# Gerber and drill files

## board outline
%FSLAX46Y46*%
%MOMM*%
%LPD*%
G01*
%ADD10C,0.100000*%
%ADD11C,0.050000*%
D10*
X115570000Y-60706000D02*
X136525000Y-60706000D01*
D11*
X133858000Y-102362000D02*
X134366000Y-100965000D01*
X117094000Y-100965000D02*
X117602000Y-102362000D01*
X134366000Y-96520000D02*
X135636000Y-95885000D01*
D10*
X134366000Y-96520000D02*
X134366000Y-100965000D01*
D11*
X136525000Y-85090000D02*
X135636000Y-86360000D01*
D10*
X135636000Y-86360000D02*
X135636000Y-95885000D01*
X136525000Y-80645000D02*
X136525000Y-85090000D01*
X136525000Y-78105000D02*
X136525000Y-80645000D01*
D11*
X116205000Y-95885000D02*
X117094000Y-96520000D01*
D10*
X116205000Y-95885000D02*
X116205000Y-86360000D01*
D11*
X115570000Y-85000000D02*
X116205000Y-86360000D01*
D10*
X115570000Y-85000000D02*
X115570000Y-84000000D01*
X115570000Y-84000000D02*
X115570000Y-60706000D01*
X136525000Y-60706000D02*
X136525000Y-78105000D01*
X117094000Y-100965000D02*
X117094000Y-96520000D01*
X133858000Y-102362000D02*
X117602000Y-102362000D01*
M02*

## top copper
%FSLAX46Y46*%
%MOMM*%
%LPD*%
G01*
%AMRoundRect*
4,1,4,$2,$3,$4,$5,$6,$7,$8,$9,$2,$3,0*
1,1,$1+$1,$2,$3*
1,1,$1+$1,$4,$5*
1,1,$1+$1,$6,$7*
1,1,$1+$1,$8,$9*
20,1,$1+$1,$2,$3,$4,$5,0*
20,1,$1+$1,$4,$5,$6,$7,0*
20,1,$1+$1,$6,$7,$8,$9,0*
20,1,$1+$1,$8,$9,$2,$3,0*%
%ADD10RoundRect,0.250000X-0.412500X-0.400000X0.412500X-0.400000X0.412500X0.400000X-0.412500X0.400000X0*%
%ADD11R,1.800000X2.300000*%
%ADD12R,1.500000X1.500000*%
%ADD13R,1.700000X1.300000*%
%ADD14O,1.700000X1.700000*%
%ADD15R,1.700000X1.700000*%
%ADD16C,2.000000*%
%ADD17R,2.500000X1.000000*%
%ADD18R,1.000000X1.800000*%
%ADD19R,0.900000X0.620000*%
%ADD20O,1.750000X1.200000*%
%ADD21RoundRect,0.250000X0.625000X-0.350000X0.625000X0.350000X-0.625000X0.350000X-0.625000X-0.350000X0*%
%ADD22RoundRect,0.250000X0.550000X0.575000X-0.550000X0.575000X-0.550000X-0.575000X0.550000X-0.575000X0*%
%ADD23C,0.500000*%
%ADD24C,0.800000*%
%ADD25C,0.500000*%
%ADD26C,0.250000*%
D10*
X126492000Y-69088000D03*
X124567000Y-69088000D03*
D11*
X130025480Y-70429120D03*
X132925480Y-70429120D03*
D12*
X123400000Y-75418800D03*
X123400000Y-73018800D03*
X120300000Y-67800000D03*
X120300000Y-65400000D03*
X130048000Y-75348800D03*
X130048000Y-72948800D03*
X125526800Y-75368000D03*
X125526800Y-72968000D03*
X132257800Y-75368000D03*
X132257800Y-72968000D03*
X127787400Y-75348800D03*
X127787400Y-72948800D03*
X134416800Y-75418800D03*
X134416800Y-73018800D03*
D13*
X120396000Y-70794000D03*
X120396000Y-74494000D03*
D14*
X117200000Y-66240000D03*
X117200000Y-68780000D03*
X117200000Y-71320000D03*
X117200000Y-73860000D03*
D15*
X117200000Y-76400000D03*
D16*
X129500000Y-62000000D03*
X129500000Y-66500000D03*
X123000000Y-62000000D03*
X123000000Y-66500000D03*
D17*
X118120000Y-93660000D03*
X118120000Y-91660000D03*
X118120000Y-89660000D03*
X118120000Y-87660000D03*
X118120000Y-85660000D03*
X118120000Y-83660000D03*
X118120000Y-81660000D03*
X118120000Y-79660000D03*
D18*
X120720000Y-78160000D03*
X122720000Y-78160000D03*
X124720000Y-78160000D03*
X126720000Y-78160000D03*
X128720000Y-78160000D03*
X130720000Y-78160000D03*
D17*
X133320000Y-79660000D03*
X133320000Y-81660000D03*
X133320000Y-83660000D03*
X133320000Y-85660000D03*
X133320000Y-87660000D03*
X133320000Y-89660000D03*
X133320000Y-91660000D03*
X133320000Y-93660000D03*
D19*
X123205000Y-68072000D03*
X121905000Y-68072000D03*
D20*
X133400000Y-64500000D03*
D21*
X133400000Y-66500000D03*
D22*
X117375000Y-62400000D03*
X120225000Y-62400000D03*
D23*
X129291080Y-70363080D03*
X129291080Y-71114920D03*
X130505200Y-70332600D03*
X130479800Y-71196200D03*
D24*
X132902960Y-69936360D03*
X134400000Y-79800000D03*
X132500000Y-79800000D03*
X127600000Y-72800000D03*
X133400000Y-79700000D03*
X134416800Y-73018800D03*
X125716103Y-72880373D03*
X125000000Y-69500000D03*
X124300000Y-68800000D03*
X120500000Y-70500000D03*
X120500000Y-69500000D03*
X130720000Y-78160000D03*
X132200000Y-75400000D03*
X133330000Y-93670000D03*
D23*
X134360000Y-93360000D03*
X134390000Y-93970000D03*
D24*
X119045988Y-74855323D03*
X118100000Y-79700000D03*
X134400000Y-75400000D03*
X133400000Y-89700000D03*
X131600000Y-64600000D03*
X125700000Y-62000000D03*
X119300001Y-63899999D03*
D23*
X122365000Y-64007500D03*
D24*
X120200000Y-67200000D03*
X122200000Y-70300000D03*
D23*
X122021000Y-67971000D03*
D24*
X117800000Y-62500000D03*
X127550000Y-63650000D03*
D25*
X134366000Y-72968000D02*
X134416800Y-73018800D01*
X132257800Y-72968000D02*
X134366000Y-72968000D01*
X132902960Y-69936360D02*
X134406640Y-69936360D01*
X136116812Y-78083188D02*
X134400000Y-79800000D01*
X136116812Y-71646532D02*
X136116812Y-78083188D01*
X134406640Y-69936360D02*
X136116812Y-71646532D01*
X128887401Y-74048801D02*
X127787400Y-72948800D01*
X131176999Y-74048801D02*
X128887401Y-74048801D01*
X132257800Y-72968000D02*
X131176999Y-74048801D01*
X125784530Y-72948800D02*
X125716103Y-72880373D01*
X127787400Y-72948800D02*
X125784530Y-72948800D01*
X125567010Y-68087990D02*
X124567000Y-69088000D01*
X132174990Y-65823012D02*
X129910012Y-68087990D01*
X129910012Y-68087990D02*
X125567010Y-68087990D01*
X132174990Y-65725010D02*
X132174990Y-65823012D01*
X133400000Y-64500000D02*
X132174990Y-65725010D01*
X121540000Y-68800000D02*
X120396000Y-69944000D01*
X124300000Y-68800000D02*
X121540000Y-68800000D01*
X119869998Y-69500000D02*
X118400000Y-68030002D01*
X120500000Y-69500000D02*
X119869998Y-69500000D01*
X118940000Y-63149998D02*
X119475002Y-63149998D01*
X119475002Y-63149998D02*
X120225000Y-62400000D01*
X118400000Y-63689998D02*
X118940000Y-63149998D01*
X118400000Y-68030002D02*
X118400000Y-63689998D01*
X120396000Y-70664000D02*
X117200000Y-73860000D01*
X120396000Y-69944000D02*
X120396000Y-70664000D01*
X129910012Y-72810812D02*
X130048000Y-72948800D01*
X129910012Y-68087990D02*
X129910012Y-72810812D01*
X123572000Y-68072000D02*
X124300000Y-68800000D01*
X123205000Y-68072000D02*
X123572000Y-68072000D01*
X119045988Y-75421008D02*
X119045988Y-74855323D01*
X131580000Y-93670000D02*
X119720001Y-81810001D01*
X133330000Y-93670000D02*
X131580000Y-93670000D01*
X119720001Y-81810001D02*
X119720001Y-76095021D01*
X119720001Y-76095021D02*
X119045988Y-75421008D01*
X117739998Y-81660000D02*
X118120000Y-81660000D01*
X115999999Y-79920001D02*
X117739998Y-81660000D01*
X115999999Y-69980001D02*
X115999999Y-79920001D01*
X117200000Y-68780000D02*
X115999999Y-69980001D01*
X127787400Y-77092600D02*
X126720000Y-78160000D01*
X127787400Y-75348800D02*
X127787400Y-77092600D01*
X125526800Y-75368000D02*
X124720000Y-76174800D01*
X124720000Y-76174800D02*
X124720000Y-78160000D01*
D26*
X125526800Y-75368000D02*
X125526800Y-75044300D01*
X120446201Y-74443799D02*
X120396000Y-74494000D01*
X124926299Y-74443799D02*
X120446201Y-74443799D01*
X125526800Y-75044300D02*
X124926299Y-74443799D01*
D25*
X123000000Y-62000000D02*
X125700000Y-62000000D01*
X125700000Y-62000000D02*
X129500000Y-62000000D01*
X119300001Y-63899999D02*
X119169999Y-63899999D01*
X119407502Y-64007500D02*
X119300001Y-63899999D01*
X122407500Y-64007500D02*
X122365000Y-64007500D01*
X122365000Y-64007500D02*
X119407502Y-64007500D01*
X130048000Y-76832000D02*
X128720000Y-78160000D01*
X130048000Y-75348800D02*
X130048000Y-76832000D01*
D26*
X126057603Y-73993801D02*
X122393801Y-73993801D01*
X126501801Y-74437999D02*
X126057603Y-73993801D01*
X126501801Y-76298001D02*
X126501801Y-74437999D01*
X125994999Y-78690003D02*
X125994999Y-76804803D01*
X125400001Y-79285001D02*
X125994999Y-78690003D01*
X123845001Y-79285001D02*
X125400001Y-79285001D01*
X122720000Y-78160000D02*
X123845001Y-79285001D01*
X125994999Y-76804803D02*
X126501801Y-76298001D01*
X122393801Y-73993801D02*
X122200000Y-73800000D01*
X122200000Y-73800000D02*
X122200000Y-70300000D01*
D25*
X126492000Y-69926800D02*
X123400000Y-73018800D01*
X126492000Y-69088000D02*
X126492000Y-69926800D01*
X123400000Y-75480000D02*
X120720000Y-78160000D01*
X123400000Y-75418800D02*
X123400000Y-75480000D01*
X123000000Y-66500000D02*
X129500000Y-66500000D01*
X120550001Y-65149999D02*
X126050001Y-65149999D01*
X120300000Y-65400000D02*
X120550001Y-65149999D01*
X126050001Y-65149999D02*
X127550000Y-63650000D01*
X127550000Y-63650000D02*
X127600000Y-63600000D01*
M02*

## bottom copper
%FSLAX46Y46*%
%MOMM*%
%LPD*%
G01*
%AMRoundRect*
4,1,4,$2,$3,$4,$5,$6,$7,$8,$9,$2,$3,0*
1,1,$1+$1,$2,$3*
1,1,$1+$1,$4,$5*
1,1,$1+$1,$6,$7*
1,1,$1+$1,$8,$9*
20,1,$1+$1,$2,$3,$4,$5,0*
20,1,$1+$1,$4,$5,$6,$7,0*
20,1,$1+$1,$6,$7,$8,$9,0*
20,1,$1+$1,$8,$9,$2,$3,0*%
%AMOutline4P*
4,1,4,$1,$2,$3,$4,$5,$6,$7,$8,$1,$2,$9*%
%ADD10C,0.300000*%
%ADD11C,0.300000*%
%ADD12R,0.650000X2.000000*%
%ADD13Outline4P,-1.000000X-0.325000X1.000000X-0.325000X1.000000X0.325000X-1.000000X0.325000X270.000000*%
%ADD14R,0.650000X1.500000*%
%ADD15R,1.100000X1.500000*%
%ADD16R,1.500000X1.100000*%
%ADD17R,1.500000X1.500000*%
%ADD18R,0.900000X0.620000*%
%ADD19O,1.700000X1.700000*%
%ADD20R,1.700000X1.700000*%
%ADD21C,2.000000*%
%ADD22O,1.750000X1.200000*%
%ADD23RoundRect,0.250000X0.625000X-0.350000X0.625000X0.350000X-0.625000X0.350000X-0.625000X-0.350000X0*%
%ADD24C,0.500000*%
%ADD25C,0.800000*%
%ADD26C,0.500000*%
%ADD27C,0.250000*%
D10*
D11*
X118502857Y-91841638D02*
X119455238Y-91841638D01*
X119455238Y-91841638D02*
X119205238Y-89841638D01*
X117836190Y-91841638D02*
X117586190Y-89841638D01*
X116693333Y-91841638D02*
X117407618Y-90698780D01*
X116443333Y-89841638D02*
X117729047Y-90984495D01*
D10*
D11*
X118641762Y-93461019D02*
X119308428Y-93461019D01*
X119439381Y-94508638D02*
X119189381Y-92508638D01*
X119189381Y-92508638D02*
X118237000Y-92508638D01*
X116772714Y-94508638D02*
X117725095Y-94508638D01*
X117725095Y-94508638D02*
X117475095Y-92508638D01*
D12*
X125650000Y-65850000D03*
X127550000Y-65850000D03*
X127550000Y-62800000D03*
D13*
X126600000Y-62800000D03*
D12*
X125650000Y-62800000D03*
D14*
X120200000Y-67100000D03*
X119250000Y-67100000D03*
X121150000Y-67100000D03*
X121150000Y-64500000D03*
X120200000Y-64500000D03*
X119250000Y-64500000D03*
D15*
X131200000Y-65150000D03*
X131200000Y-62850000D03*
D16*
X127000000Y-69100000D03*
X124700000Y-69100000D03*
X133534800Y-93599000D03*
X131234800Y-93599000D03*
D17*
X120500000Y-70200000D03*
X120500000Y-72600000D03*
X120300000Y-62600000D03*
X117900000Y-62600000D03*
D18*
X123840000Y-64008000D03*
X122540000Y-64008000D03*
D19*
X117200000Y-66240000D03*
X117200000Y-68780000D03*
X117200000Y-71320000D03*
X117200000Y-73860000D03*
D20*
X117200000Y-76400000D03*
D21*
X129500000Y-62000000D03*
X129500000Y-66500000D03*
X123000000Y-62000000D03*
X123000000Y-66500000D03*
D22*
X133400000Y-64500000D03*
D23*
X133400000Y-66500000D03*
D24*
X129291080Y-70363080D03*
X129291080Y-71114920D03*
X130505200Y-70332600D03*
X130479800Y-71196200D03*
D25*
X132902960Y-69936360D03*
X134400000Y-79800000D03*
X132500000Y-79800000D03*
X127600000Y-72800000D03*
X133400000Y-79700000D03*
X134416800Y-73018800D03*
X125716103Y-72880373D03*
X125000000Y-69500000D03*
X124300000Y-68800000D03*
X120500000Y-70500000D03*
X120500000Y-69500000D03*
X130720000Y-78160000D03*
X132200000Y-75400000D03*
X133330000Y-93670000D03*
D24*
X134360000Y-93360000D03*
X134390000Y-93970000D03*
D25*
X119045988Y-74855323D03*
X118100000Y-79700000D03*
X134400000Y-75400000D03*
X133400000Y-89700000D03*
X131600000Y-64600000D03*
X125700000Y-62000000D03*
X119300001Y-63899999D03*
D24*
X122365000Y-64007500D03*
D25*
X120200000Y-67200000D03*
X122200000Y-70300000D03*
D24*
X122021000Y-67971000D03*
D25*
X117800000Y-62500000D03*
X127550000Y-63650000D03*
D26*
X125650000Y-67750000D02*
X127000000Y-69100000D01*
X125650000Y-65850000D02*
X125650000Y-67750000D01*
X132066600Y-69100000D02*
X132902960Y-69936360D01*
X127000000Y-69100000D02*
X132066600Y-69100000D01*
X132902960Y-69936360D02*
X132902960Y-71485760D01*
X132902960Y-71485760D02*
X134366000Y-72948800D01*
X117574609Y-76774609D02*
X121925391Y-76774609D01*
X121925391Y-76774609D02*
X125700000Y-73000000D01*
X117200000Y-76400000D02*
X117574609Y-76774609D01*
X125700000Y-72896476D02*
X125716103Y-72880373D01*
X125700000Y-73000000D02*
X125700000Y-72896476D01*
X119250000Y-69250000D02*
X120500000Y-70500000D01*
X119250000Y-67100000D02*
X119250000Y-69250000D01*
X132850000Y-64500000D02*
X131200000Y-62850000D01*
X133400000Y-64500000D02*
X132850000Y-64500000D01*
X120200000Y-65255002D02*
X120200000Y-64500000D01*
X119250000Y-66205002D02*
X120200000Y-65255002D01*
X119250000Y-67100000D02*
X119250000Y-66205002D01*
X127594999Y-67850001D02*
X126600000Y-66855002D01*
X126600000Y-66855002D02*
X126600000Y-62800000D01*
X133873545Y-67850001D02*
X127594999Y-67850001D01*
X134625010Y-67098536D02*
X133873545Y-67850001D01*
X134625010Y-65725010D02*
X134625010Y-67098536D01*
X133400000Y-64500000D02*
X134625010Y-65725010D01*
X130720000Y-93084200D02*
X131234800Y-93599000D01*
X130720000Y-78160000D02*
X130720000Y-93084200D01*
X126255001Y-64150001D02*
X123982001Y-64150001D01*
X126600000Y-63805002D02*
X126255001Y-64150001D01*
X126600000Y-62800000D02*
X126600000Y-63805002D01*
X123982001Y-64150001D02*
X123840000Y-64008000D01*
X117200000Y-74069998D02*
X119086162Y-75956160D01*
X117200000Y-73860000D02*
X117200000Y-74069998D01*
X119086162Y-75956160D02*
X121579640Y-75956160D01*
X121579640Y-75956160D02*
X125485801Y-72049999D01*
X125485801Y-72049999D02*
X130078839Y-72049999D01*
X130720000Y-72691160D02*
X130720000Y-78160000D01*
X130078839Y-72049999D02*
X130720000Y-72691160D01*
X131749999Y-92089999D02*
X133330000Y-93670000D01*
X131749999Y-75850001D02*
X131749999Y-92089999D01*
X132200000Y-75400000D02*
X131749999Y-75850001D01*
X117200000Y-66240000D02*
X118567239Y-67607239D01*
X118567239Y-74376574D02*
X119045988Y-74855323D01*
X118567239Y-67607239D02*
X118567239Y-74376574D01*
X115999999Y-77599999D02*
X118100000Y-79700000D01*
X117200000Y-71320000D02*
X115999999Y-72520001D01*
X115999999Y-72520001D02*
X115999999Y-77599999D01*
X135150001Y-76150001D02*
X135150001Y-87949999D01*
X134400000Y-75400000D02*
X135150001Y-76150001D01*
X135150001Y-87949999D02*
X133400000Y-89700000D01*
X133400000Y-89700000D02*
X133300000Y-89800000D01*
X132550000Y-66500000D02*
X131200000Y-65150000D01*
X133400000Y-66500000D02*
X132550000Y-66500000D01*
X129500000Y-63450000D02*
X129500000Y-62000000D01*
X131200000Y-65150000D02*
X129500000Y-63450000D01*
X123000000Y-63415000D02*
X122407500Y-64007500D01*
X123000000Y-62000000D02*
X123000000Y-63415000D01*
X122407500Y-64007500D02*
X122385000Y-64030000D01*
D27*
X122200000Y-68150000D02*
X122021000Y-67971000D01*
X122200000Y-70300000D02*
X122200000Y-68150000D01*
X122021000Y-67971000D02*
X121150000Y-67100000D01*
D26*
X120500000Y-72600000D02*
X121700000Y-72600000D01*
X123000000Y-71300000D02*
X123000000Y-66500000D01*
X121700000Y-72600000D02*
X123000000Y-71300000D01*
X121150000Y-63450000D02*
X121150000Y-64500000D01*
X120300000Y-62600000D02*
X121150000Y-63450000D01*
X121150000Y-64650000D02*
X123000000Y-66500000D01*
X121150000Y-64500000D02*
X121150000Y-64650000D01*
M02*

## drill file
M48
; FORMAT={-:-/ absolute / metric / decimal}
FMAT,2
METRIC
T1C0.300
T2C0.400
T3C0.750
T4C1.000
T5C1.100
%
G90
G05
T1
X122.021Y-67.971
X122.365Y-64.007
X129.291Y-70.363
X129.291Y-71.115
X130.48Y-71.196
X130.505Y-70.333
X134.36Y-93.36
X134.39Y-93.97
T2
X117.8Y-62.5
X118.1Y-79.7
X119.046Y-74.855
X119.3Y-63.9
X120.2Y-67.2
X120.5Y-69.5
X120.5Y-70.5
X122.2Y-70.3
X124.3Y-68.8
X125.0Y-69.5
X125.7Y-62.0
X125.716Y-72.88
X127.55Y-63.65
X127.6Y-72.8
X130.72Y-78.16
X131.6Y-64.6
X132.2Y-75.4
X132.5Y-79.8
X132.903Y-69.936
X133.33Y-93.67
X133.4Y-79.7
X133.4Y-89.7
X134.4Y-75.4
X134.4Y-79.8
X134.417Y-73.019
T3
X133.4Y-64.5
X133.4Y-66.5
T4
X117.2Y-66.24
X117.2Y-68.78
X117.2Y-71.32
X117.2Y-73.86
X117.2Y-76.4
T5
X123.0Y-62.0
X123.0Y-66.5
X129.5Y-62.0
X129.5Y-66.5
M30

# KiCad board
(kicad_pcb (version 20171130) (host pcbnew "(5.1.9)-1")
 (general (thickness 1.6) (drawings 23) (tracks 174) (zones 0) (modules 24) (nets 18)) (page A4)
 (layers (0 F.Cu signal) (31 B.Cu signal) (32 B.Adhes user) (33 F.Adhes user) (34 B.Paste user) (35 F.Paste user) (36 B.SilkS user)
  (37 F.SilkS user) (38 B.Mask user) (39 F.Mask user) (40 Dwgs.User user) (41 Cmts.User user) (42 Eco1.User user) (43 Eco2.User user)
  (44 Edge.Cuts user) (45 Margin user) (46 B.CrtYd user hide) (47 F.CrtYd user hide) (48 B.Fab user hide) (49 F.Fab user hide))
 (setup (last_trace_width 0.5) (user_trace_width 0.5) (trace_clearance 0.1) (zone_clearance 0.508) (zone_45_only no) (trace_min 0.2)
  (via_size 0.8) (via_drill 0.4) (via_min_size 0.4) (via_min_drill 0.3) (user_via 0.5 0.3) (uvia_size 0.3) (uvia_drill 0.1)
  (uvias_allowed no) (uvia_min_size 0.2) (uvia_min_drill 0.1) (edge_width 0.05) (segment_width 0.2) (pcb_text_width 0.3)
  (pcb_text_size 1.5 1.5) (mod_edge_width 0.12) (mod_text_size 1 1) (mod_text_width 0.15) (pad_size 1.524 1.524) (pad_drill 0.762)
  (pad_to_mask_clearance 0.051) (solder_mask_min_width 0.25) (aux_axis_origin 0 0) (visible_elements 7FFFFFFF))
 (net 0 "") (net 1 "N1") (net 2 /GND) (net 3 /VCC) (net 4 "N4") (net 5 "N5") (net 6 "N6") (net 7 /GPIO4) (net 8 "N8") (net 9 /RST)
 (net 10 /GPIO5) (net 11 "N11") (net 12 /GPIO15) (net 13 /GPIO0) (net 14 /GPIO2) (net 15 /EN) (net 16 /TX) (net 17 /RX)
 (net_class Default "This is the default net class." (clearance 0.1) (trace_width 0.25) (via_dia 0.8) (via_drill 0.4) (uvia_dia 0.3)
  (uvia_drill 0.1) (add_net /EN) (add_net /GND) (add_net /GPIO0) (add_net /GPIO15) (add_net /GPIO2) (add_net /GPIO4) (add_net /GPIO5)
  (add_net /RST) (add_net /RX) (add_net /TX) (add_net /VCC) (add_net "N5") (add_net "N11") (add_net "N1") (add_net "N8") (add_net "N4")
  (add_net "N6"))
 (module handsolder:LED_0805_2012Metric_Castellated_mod (layer F.Cu) (at 125.5295 69.088)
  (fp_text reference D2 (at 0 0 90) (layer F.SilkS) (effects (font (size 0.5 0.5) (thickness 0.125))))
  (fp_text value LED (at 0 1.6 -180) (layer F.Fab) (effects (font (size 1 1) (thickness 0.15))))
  (pad 2 smd roundrect (at 0.9625 0) (size 1.325 1.3) (layers F.Cu F.Paste F.Mask) (roundrect_rratio 0.1923076923076923) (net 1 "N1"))
  (pad 1 smd roundrect (at -0.9625 0) (size 1.325 1.3) (layers F.Cu F.Paste F.Mask) (roundrect_rratio 0.1923076923076923) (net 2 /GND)))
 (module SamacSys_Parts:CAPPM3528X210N (layer F.Cu) (at 131.47548 70.42912 180)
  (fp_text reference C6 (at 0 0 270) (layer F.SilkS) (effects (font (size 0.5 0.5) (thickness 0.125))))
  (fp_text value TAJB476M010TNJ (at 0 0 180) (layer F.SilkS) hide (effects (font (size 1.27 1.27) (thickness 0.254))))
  (pad 2 smd rect (at 1.45 0 180) (size 1.8 2.3) (layers F.Cu F.Paste F.Mask) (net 2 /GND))
  (pad 1 smd rect (at -1.45 0 180) (size 1.8 2.3) (layers F.Cu F.Paste F.Mask) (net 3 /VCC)))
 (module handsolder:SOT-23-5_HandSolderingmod (layer B.Cu) (at 126.6 64.35 270)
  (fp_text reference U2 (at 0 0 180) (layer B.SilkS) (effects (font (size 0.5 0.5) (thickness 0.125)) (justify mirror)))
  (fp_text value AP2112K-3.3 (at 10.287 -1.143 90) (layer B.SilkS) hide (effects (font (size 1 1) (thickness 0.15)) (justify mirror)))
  (pad 5 smd rect (at 1.5 0.95 270) (size 2 0.65) (layers B.Cu B.Paste B.Mask) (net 3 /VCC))
  (pad 4 smd rect (at 1.5 -0.95 270) (size 2 0.65) (layers B.Cu B.Paste B.Mask))
  (pad 3 smd rect (at -1.55 -0.95 270) (size 2 0.65) (layers B.Cu B.Paste B.Mask) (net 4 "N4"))
  (pad 2 smd trapezoid (at -1.55 0 270) (size 2 0.65) (layers B.Cu B.Paste B.Mask) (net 2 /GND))
  (pad 1 smd rect (at -1.55 0.95 270) (size 2 0.65) (layers B.Cu B.Paste B.Mask) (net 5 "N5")))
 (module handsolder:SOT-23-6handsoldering (layer B.Cu) (at 120.2 65.8 270)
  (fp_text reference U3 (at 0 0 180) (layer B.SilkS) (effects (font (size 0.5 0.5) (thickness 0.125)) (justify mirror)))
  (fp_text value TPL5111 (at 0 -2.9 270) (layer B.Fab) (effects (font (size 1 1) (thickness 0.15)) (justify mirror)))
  (pad 5 smd rect (at 1.3 0 270) (size 1.5 0.65) (layers B.Cu B.Paste B.Mask) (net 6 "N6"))
  (pad 6 smd rect (at 1.3 0.95 270) (size 1.5 0.65) (layers B.Cu B.Paste B.Mask) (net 2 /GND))
  (pad 4 smd rect (at 1.3 -0.95 270) (size 1.5 0.65) (layers B.Cu B.Paste B.Mask) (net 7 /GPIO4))
  (pad 3 smd rect (at -1.3 -0.95 270) (size 1.5 0.65) (layers B.Cu B.Paste B.Mask) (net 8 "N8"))
  (pad 2 smd rect (at -1.3 0 270) (size 1.5 0.65) (layers B.Cu B.Paste B.Mask) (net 2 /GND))
  (pad 1 smd rect (at -1.3 0.95 270) (size 1.5 0.65) (layers B.Cu B.Paste B.Mask) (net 5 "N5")))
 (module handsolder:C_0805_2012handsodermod (layer B.Cu) (at 131.2 64 270)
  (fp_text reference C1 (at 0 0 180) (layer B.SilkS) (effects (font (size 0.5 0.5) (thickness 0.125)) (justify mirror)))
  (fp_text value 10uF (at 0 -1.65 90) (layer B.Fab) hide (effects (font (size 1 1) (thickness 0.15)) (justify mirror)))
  (pad 2 smd rect (at 1.15 0 270) (size 1.5 1.1) (layers B.Cu B.Paste B.Mask) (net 5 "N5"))
  (pad 1 smd rect (at -1.15 0 270) (size 1.5 1.1) (layers B.Cu B.Paste B.Mask) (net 2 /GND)))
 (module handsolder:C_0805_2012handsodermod (layer B.Cu) (at 125.85 69.1)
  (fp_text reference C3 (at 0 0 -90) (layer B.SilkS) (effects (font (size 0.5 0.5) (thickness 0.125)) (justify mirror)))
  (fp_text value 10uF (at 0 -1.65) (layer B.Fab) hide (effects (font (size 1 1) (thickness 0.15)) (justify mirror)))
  (pad 2 smd rect (at 1.15 0) (size 1.5 1.1) (layers B.Cu B.Paste B.Mask) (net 3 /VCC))
  (pad 1 smd rect (at -1.15 0) (size 1.5 1.1) (layers B.Cu B.Paste B.Mask) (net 2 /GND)))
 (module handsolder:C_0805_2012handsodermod (layer B.Cu) (at 132.3848 93.599)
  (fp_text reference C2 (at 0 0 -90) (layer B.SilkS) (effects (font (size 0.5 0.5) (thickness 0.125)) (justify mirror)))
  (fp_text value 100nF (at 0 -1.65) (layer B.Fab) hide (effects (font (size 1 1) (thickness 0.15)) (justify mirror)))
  (pad 2 smd rect (at 1.15 0) (size 1.5 1.1) (layers B.Cu B.Paste B.Mask) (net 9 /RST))
  (pad 1 smd rect (at -1.15 0) (size 1.5 1.1) (layers B.Cu B.Paste B.Mask) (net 2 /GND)))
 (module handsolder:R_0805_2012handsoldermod (layer B.Cu) (at 120.5 71.4 90)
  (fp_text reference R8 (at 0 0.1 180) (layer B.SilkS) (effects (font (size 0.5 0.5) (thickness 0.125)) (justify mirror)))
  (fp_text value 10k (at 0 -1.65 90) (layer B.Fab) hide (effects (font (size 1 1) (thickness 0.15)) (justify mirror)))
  (pad 2 smd rect (at 1.2 0 90) (size 1.5 1.5) (layers B.Cu B.Paste B.Mask) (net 2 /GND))
  (pad 1 smd rect (at -1.2 0 90) (size 1.5 1.5) (layers B.Cu B.Paste B.Mask) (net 8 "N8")))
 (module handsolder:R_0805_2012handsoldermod (layer F.Cu) (at 123.4 74.2188 270)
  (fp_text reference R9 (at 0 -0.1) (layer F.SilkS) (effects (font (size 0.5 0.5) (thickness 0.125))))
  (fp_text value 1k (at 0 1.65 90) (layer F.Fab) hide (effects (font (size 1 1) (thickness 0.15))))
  (pad 2 smd rect (at 1.2 0 270) (size 1.5 1.5) (layers F.Cu F.Paste F.Mask) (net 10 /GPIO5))
  (pad 1 smd rect (at -1.2 0 270) (size 1.5 1.5) (layers F.Cu F.Paste F.Mask) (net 1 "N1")))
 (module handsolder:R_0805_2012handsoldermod (layer F.Cu) (at 120.3 66.6 270)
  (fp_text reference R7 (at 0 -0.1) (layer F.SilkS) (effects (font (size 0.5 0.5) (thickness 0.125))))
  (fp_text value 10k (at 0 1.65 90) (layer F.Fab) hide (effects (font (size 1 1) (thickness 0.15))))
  (pad 2 smd rect (at 1.2 0 270) (size 1.5 1.5) (layers F.Cu F.Paste F.Mask) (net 6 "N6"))
  (pad 1 smd rect (at -1.2 0 270) (size 1.5 1.5) (layers F.Cu F.Paste F.Mask) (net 4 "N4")))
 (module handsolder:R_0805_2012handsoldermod (layer B.Cu) (at 119.1 62.6)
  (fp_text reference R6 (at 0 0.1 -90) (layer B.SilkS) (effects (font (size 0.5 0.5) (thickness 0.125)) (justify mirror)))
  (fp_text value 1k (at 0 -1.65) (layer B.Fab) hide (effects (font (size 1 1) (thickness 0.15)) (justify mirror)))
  (pad 2 smd rect (at 1.2 0) (size 1.5 1.5) (layers B.Cu B.Paste B.Mask) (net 8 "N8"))
  (pad 1 smd rect (at -1.2 0) (size 1.5 1.5) (layers B.Cu B.Paste B.Mask) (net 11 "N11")))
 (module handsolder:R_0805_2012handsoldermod (layer F.Cu) (at 130.048 74.1488 270)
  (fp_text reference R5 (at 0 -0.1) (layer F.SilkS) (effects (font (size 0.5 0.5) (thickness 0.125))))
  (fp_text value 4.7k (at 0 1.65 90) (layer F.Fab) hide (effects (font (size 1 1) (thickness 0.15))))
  (pad 2 smd rect (at 1.2 0 270) (size 1.5 1.5) (layers F.Cu F.Paste F.Mask) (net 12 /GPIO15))
  (pad 1 smd rect (at -1.2 0 270) (size 1.5 1.5) (layers F.Cu F.Paste F.Mask) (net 2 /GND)))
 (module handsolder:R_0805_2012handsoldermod (layer F.Cu) (at 125.5268 74.168 270)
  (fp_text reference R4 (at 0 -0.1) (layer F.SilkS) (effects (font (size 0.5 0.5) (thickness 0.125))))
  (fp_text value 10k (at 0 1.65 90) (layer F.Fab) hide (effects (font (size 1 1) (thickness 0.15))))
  (pad 2 smd rect (at 1.2 0 270) (size 1.5 1.5) (layers F.Cu F.Paste F.Mask) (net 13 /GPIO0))
  (pad 1 smd rect (at -1.2 0 270) (size 1.5 1.5) (layers F.Cu F.Paste F.Mask) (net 3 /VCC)))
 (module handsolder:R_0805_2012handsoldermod (layer F.Cu) (at 132.2578 74.168 270)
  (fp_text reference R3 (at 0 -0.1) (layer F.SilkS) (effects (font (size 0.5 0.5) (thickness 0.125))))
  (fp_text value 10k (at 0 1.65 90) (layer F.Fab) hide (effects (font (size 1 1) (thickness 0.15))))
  (pad 2 smd rect (at 1.2 0 270) (size 1.5 1.5) (layers F.Cu F.Paste F.Mask) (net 9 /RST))
  (pad 1 smd rect (at -1.2 0 270) (size 1.5 1.5) (layers F.Cu F.Paste F.Mask) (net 3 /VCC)))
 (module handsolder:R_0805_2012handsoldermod (layer F.Cu) (at 127.7874 74.1488 270)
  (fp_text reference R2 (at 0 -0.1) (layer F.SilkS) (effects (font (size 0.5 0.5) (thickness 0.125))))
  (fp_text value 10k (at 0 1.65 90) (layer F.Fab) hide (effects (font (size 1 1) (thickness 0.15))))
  (pad 2 smd rect (at 1.2 0 270) (size 1.5 1.5) (layers F.Cu F.Paste F.Mask) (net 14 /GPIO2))
  (pad 1 smd rect (at -1.2 0 270) (size 1.5 1.5) (layers F.Cu F.Paste F.Mask) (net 3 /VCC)))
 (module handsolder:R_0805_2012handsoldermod (layer F.Cu) (at 134.4168 74.2188 270)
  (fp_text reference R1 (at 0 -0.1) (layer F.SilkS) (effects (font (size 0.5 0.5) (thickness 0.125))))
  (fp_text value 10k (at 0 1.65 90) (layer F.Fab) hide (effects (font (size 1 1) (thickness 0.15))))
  (pad 2 smd rect (at 1.2 0 270) (size 1.5 1.5) (layers F.Cu F.Paste F.Mask) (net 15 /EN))
  (pad 1 smd rect (at -1.2 0 270) (size 1.5 1.5) (layers F.Cu F.Paste F.Mask) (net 3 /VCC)))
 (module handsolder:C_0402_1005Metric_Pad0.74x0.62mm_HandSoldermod (layer B.Cu) (at 123.19 64.008)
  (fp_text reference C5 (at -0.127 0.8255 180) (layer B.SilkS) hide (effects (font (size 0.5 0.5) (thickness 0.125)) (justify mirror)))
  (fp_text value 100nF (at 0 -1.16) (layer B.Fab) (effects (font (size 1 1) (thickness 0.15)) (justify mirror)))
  (pad 2 smd rect (at 0.65 0) (size 0.9 0.62) (layers B.Cu B.Paste B.Mask) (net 2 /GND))
  (pad 1 smd rect (at -0.65 0) (size 0.9 0.62) (layers B.Cu B.Paste B.Mask) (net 5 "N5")))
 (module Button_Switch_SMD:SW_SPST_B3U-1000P (layer F.Cu) (at 120.396 72.644 90)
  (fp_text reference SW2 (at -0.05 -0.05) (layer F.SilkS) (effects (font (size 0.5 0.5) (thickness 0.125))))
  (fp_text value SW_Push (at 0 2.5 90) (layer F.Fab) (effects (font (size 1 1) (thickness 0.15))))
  (pad 2 smd rect (at 1.85 0 90) (size 1.3 1.7) (layers F.Cu F.Paste F.Mask) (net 2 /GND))
  (pad 1 smd rect (at -1.85 0 90) (size 1.3 1.7) (layers F.Cu F.Paste F.Mask) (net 13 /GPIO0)))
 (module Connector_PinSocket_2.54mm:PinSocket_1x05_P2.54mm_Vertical (layer F.Cu) (at 117.2 76.4 180)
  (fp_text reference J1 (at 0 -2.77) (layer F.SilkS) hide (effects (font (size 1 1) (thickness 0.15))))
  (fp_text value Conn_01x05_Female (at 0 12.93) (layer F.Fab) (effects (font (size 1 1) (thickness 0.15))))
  (pad 5 thru_hole oval (at 0 10.16 180) (size 1.7 1.7) (drill 1) (layers *.Cu *.Mask) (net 9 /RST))
  (pad 4 thru_hole oval (at 0 7.62 180) (size 1.7 1.7) (drill 1) (layers *.Cu *.Mask) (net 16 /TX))
  (pad 3 thru_hole oval (at 0 5.08 180) (size 1.7 1.7) (drill 1) (layers *.Cu *.Mask) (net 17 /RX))
  (pad 2 thru_hole oval (at 0 2.54 180) (size 1.7 1.7) (drill 1) (layers *.Cu *.Mask) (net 2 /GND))
  (pad 1 thru_hole rect (at 0 0 180) (size 1.7 1.7) (drill 1) (layers *.Cu *.Mask) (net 3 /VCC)))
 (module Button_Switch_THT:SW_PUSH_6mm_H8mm (layer F.Cu) (at 123 62)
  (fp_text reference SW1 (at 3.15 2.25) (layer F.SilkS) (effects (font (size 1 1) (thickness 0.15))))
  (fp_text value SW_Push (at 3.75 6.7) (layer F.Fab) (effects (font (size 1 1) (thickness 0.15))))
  (pad 1 thru_hole circle (at 6.5 0 90) (size 2 2) (drill 1.1) (layers *.Cu *.Mask) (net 5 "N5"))
  (pad 2 thru_hole circle (at 6.5 4.5 90) (size 2 2) (drill 1.1) (layers *.Cu *.Mask) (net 8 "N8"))
  (pad 1 thru_hole circle (at 0 0 90) (size 2 2) (drill 1.1) (layers *.Cu *.Mask) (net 5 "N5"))
  (pad 2 thru_hole circle (at 0 4.5 90) (size 2 2) (drill 1.1) (layers *.Cu *.Mask) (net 8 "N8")))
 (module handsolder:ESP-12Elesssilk (layer F.Cu) (at 125.72 90.16 180)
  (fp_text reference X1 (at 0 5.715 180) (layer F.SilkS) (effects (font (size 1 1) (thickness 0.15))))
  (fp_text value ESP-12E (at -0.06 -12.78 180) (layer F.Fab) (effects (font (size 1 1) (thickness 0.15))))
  (pad 22 smd rect (at 7.6 -3.5 180) (size 2.5 1) (layers F.Cu F.Paste F.Mask))
  (pad 21 smd rect (at 7.6 -1.5 180) (size 2.5 1) (layers F.Cu F.Paste F.Mask))
  (pad 20 smd rect (at 7.6 0.5 180) (size 2.5 1) (layers F.Cu F.Paste F.Mask))
  (pad 19 smd rect (at 7.6 2.5 180) (size 2.5 1) (layers F.Cu F.Paste F.Mask))
  (pad 18 smd rect (at 7.6 4.5 180) (size 2.5 1) (layers F.Cu F.Paste F.Mask))
  (pad 17 smd rect (at 7.6 6.5 180) (size 2.5 1) (layers F.Cu F.Paste F.Mask))
  (pad 16 smd rect (at 7.6 8.5 180) (size 2.5 1) (layers F.Cu F.Paste F.Mask) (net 16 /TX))
  (pad 15 smd rect (at 7.6 10.5 180) (size 2.5 1) (layers F.Cu F.Paste F.Mask) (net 17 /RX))
  (pad 14 smd rect (at 5 12 180) (size 1 1.8) (layers F.Cu F.Paste F.Mask) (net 10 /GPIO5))
  (pad 13 smd rect (at 3 12 180) (size 1 1.8) (layers F.Cu F.Paste F.Mask) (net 7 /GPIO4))
  (pad 12 smd rect (at 1 12 180) (size 1 1.8) (layers F.Cu F.Paste F.Mask) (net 13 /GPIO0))
  (pad 11 smd rect (at -1 12 180) (size 1 1.8) (layers F.Cu F.Paste F.Mask) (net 14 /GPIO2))
  (pad 10 smd rect (at -3 12 180) (size 1 1.8) (layers F.Cu F.Paste F.Mask) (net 12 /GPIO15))
  (pad 9 smd rect (at -5 12 180) (size 1 1.8) (layers F.Cu F.Paste F.Mask) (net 2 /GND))
  (pad 8 smd rect (at -7.6 10.5 180) (size 2.5 1) (layers F.Cu F.Paste F.Mask) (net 3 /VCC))
  (pad 7 smd rect (at -7.6 8.5 180) (size 2.5 1) (layers F.Cu F.Paste F.Mask))
  (pad 6 smd rect (at -7.6 6.5 180) (size 2.5 1) (layers F.Cu F.Paste F.Mask))
  (pad 5 smd rect (at -7.6 4.5 180) (size 2.5 1) (layers F.Cu F.Paste F.Mask))
  (pad 4 smd rect (at -7.6 2.5 180) (size 2.5 1) (layers F.Cu F.Paste F.Mask))
  (pad 3 smd rect (at -7.6 0.5 180) (size 2.5 1) (layers F.Cu F.Paste F.Mask) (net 15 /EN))
  (pad 2 smd rect (at -7.6 -1.5 180) (size 2.5 1) (layers F.Cu F.Paste F.Mask))
  (pad 1 smd rect (at -7.6 -3.5 180) (size 2.5 1) (layers F.Cu F.Paste F.Mask) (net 9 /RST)))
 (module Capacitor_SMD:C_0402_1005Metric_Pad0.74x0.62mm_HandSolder (layer F.Cu) (at 122.555 68.072)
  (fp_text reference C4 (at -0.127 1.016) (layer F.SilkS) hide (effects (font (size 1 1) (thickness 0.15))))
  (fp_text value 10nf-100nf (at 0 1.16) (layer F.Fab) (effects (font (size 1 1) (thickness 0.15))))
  (pad 2 smd rect (at 0.65 0) (size 0.9 0.62) (layers F.Cu F.Paste F.Mask) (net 2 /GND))
  (pad 1 smd rect (at -0.65 0) (size 0.9 0.62) (layers F.Cu F.Paste F.Mask) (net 7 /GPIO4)))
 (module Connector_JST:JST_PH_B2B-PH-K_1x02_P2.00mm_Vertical (layer F.Cu) (at 133.4 66.5 90)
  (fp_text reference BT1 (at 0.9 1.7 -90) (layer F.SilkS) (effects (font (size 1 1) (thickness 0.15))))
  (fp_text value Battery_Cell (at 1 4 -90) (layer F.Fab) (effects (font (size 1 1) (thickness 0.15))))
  (pad 2 thru_hole oval (at 2 0 90) (size 1.2 1.75) (drill 0.75) (layers *.Cu *.Mask) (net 2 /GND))
  (pad 1 thru_hole roundrect (at 0 0 90) (size 1.2 1.75) (drill 0.75) (layers *.Cu *.Mask) (roundrect_rratio 0.208333) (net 5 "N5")))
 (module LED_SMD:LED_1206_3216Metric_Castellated (layer F.Cu) (at 118.8 62.4 180)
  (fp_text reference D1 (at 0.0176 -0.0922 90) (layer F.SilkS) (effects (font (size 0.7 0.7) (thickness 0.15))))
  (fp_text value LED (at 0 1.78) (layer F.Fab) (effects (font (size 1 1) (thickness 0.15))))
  (pad 2 smd roundrect (at 1.425 0 180) (size 1.6 1.65) (layers F.Cu F.Paste F.Mask) (roundrect_rratio 0.15625) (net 11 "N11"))
  (pad 1 smd roundrect (at -1.425 0 180) (size 1.6 1.65) (layers F.Cu F.Paste F.Mask) (roundrect_rratio 0.15625) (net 2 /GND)))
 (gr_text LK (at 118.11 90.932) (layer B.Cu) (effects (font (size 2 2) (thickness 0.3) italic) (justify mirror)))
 (gr_line (start 115.57 60.706) (end 136.525 60.706) (layer Edge.Cuts) (width 0.1))
 (gr_line (start 133.858 102.362) (end 134.366 100.965) (layer Edge.Cuts) (width 0.05))
 (gr_line (start 117.094 100.965) (end 117.602 102.362) (layer Edge.Cuts) (width 0.05))
 (gr_line (start 134.366 96.52) (end 135.636 95.885) (layer Edge.Cuts) (width 0.05))
 (gr_line (start 134.366 96.52) (end 134.366 100.965) (layer Edge.Cuts) (width 0.1))
 (gr_line (start 136.525 85.09) (end 135.636 86.36) (layer Edge.Cuts) (width 0.05))
 (gr_line (start 135.636 86.36) (end 135.636 95.885) (layer Edge.Cuts) (width 0.1))
 (gr_line (start 136.525 80.645) (end 136.525 85.09) (layer Edge.Cuts) (width 0.1))
 (gr_line (start 136.525 78.105) (end 136.525 80.645) (layer Edge.Cuts) (width 0.1))
 (gr_line (start 116.205 95.885) (end 117.094 96.52) (layer Edge.Cuts) (width 0.05))
 (gr_line (start 116.205 95.885) (end 116.205 86.36) (layer Edge.Cuts) (width 0.1))
 (gr_line (start 115.57 85) (end 116.205 86.36) (layer Edge.Cuts) (width 0.05))
 (gr_line (start 115.57 85) (end 115.57 84) (layer Edge.Cuts) (width 0.1))
 (gr_line (start 115.57 84) (end 115.57 60.706) (layer Edge.Cuts) (width 0.1))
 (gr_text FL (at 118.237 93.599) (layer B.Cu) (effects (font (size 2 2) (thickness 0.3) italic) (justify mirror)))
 (gr_line (start 136.525 60.706) (end 136.525 78.105) (layer Edge.Cuts) (width 0.1))
 (gr_line (start 117.094 100.965) (end 117.094 96.52) (layer Edge.Cuts) (width 0.1))
 (gr_line (start 133.858 102.362) (end 117.602 102.362) (layer Edge.Cuts) (width 0.1))
 (via (at 129.29108 70.36308) (size 0.5) (drill 0.3) (layers F.Cu B.Cu) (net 2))
 (via (at 129.29108 71.11492) (size 0.5) (drill 0.3) (layers F.Cu B.Cu) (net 2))
 (via (at 130.5052 70.3326) (size 0.5) (drill 0.3) (layers F.Cu B.Cu) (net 2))
 (via (at 130.4798 71.1962) (size 0.5) (drill 0.3) (layers F.Cu B.Cu) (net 2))
 (via (at 132.90296 69.93636) (size 0.8) (drill 0.4) (layers F.Cu B.Cu) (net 3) (status 30))
 (via (at 134.4 79.8) (size 0.8) (drill 0.4) (layers F.Cu B.Cu) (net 3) (status 30))
 (via (at 132.5 79.8) (size 0.8) (drill 0.4) (layers F.Cu B.Cu) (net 3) (status 30))
 (segment (start 125.65 67.75) (end 127 69.1) (width 0.5) (layer B.Cu) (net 3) (status 20))
 (segment (start 125.65 65.85) (end 125.65 67.75) (width 0.5) (layer B.Cu) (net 3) (status 10))
 (segment (start 134.366 72.968) (end 134.4168 73.0188) (width 0.5) (layer F.Cu) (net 3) (status 30))
 (segment (start 132.2578 72.968) (end 134.366 72.968) (width 0.5) (layer F.Cu) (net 3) (status 30))
 (via (at 127.6 72.8) (size 0.8) (drill 0.4) (layers F.Cu B.Cu) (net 3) (status 30))
 (via (at 133.4 79.7) (size 0.8) (drill 0.4) (layers F.Cu B.Cu) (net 3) (status 30))
 (segment (start 132.0666 69.1) (end 132.90296 69.93636) (width 0.5) (layer B.Cu) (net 3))
 (segment (start 127 69.1) (end 132.0666 69.1) (width 0.5) (layer B.Cu) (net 3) (status 10))
 (segment (start 132.90296 69.93636) (end 132.90296 71.48576) (width 0.5) (layer B.Cu) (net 3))
 (segment (start 132.90296 71.48576) (end 134.366 72.9488) (width 0.5) (layer B.Cu) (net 3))
 (via (at 134.4168 73.0188) (size 0.8) (drill 0.4) (layers F.Cu B.Cu) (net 3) (status 30))
 (segment (start 132.90296 69.93636) (end 134.40664 69.93636) (width 0.5) (layer F.Cu) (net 3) (status 10))
 (segment (start 136.116812 78.083188) (end 134.4 79.8) (width 0.5) (layer F.Cu) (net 3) (status 20))
 (segment (start 136.116812 71.646532) (end 136.116812 78.083188) (width 0.5) (layer F.Cu) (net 3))
 (segment (start 134.40664 69.93636) (end 136.116812 71.646532) (width 0.5) (layer F.Cu) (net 3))
 (segment (start 128.887401 74.048801) (end 127.7874 72.9488) (width 0.5) (layer F.Cu) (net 3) (status 20))
 (segment (start 131.176999 74.048801) (end 128.887401 74.048801) (width 0.5) (layer F.Cu) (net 3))
 (segment (start 132.2578 72.968) (end 131.176999 74.048801) (width 0.5) (layer F.Cu) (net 3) (status 10))
 (via (at 125.716103 72.880373) (size 0.8) (drill 0.4) (layers F.Cu B.Cu) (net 3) (status 30))
 (segment (start 117.574609 76.774609) (end 121.925391 76.774609) (width 0.5) (layer B.Cu) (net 3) (status 10))
 (segment (start 121.925391 76.774609) (end 125.7 73) (width 0.5) (layer B.Cu) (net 3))
 (segment (start 117.2 76.4) (end 117.574609 76.774609) (width 0.5) (layer B.Cu) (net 3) (status 30))
 (segment (start 125.7 72.896476) (end 125.716103 72.880373) (width 0.5) (layer B.Cu) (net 3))
 (segment (start 125.7 73) (end 125.7 72.896476) (width 0.5) (layer B.Cu) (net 3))
 (segment (start 125.78453 72.9488) (end 125.716103 72.880373) (width 0.5) (layer F.Cu) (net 3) (status 30))
 (segment (start 127.7874 72.9488) (end 125.78453 72.9488) (width 0.5) (layer F.Cu) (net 3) (status 30))
 (via (at 125 69.5) (size 0.8) (drill 0.4) (layers F.Cu B.Cu) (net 2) (status 30))
 (via (at 124.3 68.8) (size 0.8) (drill 0.4) (layers F.Cu B.Cu) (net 2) (status 30))
 (via (at 120.5 70.5) (size 0.8) (drill 0.4) (layers F.Cu B.Cu) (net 2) (status 30))
 (via (at 120.5 69.5) (size 0.8) (drill 0.4) (layers F.Cu B.Cu) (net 2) (status 30))
 (segment (start 119.25 69.25) (end 120.5 70.5) (width 0.5) (layer B.Cu) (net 2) (status 20))
 (segment (start 119.25 67.1) (end 119.25 69.25) (width 0.5) (layer B.Cu) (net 2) (status 10))
 (segment (start 132.85 64.5) (end 131.2 62.85) (width 0.5) (layer B.Cu) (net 2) (status 30))
 (segment (start 133.4 64.5) (end 132.85 64.5) (width 0.5) (layer B.Cu) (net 2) (status 30))
 (segment (start 120.2 65.255002) (end 120.2 64.5) (width 0.5) (layer B.Cu) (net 2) (status 20))
 (segment (start 119.25 66.205002) (end 120.2 65.255002) (width 0.5) (layer B.Cu) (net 2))
 (segment (start 119.25 67.1) (end 119.25 66.205002) (width 0.5) (layer B.Cu) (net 2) (status 10))
 (segment (start 127.594999 67.850001) (end 126.6 66.855002) (width 0.5) (layer B.Cu) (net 2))
 (segment (start 126.6 66.855002) (end 126.6 62.8) (width 0.5) (layer B.Cu) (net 2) (status 20))
 (segment (start 133.873545 67.850001) (end 127.594999 67.850001) (width 0.5) (layer B.Cu) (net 2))
 (segment (start 134.62501 67.098536) (end 133.873545 67.850001) (width 0.5) (layer B.Cu) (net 2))
 (segment (start 134.62501 65.72501) (end 134.62501 67.098536) (width 0.5) (layer B.Cu) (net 2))
 (segment (start 133.4 64.5) (end 134.62501 65.72501) (width 0.5) (layer B.Cu) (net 2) (status 10))
 (segment (start 125.56701 68.08799) (end 124.567 69.088) (width 0.5) (layer F.Cu) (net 2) (status 20))
 (segment (start 132.17499 65.823012) (end 129.910012 68.08799) (width 0.5) (layer F.Cu) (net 2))
 (segment (start 129.910012 68.08799) (end 125.56701 68.08799) (width 0.5) (layer F.Cu) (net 2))
 (segment (start 132.17499 65.72501) (end 132.17499 65.823012) (width 0.5) (layer F.Cu) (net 2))
 (segment (start 133.4 64.5) (end 132.17499 65.72501) (width 0.5) (layer F.Cu) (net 2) (status 10))
 (segment (start 121.54 68.8) (end 120.396 69.944) (width 0.5) (layer F.Cu) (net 2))
 (segment (start 124.3 68.8) (end 121.54 68.8) (width 0.5) (layer F.Cu) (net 2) (status 10))
 (segment (start 119.869998 69.5) (end 118.4 68.030002) (width 0.5) (layer F.Cu) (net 2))
 (segment (start 120.5 69.5) (end 119.869998 69.5) (width 0.5) (layer F.Cu) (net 2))
 (segment (start 118.94 63.149998) (end 119.475002 63.149998) (width 0.5) (layer F.Cu) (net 2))
 (segment (start 119.475002 63.149998) (end 120.225 62.4) (width 0.5) (layer F.Cu) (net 2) (status 20))
 (segment (start 118.4 63.689998) (end 118.94 63.149998) (width 0.5) (layer F.Cu) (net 2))
 (segment (start 118.4 68.030002) (end 118.4 63.689998) (width 0.5) (layer F.Cu) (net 2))
 (segment (start 120.396 70.664) (end 117.2 73.86) (width 0.5) (layer F.Cu) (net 2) (status 30))
 (segment (start 120.396 69.944) (end 120.396 70.664) (width 0.5) (layer F.Cu) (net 2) (status 20))
 (segment (start 129.910012 72.810812) (end 130.048 72.9488) (width 0.5) (layer F.Cu) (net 2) (status 30))
 (segment (start 129.910012 68.08799) (end 129.910012 72.810812) (width 0.5) (layer F.Cu) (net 2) (status 20))
 (via (at 130.72 78.16) (size 0.8) (drill 0.4) (layers F.Cu B.Cu) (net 2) (status 30))
 (segment (start 130.72 93.0842) (end 131.2348 93.599) (width 0.5) (layer B.Cu) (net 2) (status 30))
 (segment (start 130.72 78.16) (end 130.72 93.0842) (width 0.5) (layer B.Cu) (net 2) (status 20))
 (segment (start 123.572 68.072) (end 124.3 68.8) (width 0.5) (layer F.Cu) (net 2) (status 30))
 (segment (start 123.205 68.072) (end 123.572 68.072) (width 0.5) (layer F.Cu) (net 2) (status 30))
 (segment (start 126.255001 64.150001) (end 123.982001 64.150001) (width 0.5) (layer B.Cu) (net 2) (status 20))
 (segment (start 126.6 63.805002) (end 126.255001 64.150001) (width 0.5) (layer B.Cu) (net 2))
 (segment (start 126.6 62.8) (end 126.6 63.805002) (width 0.5) (layer B.Cu) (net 2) (status 10))
 (segment (start 123.982001 64.150001) (end 123.84 64.008) (width 0.5) (layer B.Cu) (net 2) (status 30))
 (segment (start 117.2 74.069998) (end 119.086162 75.95616) (width 0.5) (layer B.Cu) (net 2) (status 10))
 (segment (start 117.2 73.86) (end 117.2 74.069998) (width 0.5) (layer B.Cu) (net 2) (status 30))
 (segment (start 119.086162 75.95616) (end 121.57964 75.95616) (width 0.5) (layer B.Cu) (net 2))
 (segment (start 121.57964 75.95616) (end 125.485801 72.049999) (width 0.5) (layer B.Cu) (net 2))
 (segment (start 125.485801 72.049999) (end 130.078839 72.049999) (width 0.5) (layer B.Cu) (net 2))
 (segment (start 130.72 72.69116) (end 130.72 78.16) (width 0.5) (layer B.Cu) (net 2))
 (segment (start 130.078839 72.049999) (end 130.72 72.69116) (width 0.5) (layer B.Cu) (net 2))
 (via (at 132.2 75.4) (size 0.8) (drill 0.4) (layers F.Cu B.Cu) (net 9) (status 30))
 (via (at 133.33 93.67) (size 0.8) (drill 0.4) (layers F.Cu B.Cu) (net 9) (status 30))
 (via (at 134.36 93.36) (size 0.5) (drill 0.3) (layers F.Cu B.Cu) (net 9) (status 30))
 (via (at 134.39 93.97) (size 0.5) (drill 0.3) (layers F.Cu B.Cu) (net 9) (status 30))
 (segment (start 131.749999 92.089999) (end 133.33 93.67) (width 0.5) (layer B.Cu) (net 9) (status 20))
 (segment (start 131.749999 75.850001) (end 131.749999 92.089999) (width 0.5) (layer B.Cu) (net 9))
 (segment (start 132.2 75.4) (end 131.749999 75.850001) (width 0.5) (layer B.Cu) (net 9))
 (segment (start 119.045988 75.421008) (end 119.045988 74.855323) (width 0.5) (layer F.Cu) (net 9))
 (segment (start 131.58 93.67) (end 119.720001 81.810001) (width 0.5) (layer F.Cu) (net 9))
 (segment (start 133.33 93.67) (end 131.58 93.67) (width 0.5) (layer F.Cu) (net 9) (status 10))
 (segment (start 117.2 66.24) (end 118.567239 67.607239) (width 0.5) (layer B.Cu) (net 9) (status 10))
 (via (at 119.045988 74.855323) (size 0.8) (drill 0.4) (layers F.Cu B.Cu) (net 9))
 (segment (start 118.567239 74.376574) (end 119.045988 74.855323) (width 0.5) (layer B.Cu) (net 9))
 (segment (start 118.567239 67.607239) (end 118.567239 74.376574) (width 0.5) (layer B.Cu) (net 9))
 (segment (start 119.720001 81.810001) (end 119.720001 76.095021) (width 0.5) (layer F.Cu) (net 9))
 (segment (start 119.720001 76.095021) (end 119.045988 75.421008) (width 0.5) (layer F.Cu) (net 9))
 (via (at 118.1 79.7) (size 0.8) (drill 0.4) (layers F.Cu B.Cu) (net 17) (status 30))
 (segment (start 115.999999 77.599999) (end 118.1 79.7) (width 0.5) (layer B.Cu) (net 17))
 (segment (start 117.2 71.32) (end 115.999999 72.520001) (width 0.5) (layer B.Cu) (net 17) (status 10))
 (segment (start 115.999999 72.520001) (end 115.999999 77.599999) (width 0.5) (layer B.Cu) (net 17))
 (segment (start 117.739998 81.66) (end 118.12 81.66) (width 0.5) (layer F.Cu) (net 16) (status 30))
 (segment (start 115.999999 79.920001) (end 117.739998 81.66) (width 0.5) (layer F.Cu) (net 16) (status 20))
 (segment (start 115.999999 69.980001) (end 115.999999 79.920001) (width 0.5) (layer F.Cu) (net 16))
 (segment (start 117.2 68.78) (end 115.999999 69.980001) (width 0.5) (layer F.Cu) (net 16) (status 10))
 (via (at 134.4 75.4) (size 0.8) (drill 0.4) (layers F.Cu B.Cu) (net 15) (status 30))
 (segment (start 135.150001 76.150001) (end 135.150001 87.949999) (width 0.5) (layer B.Cu) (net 15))
 (segment (start 134.4 75.4) (end 135.150001 76.150001) (width 0.5) (layer B.Cu) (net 15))
 (segment (start 135.150001 87.949999) (end 133.4 89.7) (width 0.5) (layer B.Cu) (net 15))
 (segment (start 133.4 89.7) (end 133.3 89.8) (width 0.5) (layer B.Cu) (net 15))
 (via (at 133.4 89.7) (size 0.8) (drill 0.4) (layers F.Cu B.Cu) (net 15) (status 30))
 (segment (start 127.7874 77.0926) (end 126.72 78.16) (width 0.5) (layer F.Cu) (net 14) (status 20))
 (segment (start 127.7874 75.3488) (end 127.7874 77.0926) (width 0.5) (layer F.Cu) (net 14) (status 10))
 (segment (start 125.5268 75.368) (end 124.72 76.1748) (width 0.5) (layer F.Cu) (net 13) (status 10))
 (segment (start 124.72 76.1748) (end 124.72 78.16) (width 0.5) (layer F.Cu) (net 13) (status 20))
 (segment (start 125.5268 75.368) (end 125.5268 75.0443) (width 0.25) (layer F.Cu) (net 13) (status 30))
 (segment (start 120.446201 74.443799) (end 120.396 74.494) (width 0.25) (layer F.Cu) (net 13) (status 30))
 (segment (start 124.926299 74.443799) (end 120.446201 74.443799) (width 0.25) (layer F.Cu) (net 13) (status 20))
 (segment (start 125.5268 75.0443) (end 124.926299 74.443799) (width 0.25) (layer F.Cu) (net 13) (status 10))
 (via (at 131.6 64.6) (size 0.8) (drill 0.4) (layers F.Cu B.Cu) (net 5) (status 30))
 (segment (start 123 62) (end 125.7 62) (width 0.5) (layer F.Cu) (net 5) (status 10))
 (segment (start 125.7 62) (end 129.5 62) (width 0.5) (layer F.Cu) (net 5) (status 20))
 (via (at 125.7 62) (size 0.8) (drill 0.4) (layers F.Cu B.Cu) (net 5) (status 30))
 (segment (start 132.55 66.5) (end 131.2 65.15) (width 0.5) (layer B.Cu) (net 5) (status 30))
 (segment (start 133.4 66.5) (end 132.55 66.5) (width 0.5) (layer B.Cu) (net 5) (status 30))
 (segment (start 129.5 63.45) (end 129.5 62) (width 0.5) (layer B.Cu) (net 5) (status 20))
 (segment (start 131.2 65.15) (end 129.5 63.45) (width 0.5) (layer B.Cu) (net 5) (status 10))
 (segment (start 119.300001 63.899999) (end 119.169999 63.899999) (width 0.5) (layer F.Cu) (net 5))
 (via (at 119.300001 63.899999) (size 0.8) (drill 0.4) (layers F.Cu B.Cu) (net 5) (status 30))
 (segment (start 123 63.415) (end 122.4075 64.0075) (width 0.5) (layer B.Cu) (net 5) (status 20))
 (segment (start 123 62) (end 123 63.415) (width 0.5) (layer B.Cu) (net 5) (status 10))
 (segment (start 122.4075 64.0075) (end 122.385 64.03) (width 0.5) (layer B.Cu) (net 5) (status 30))
 (segment (start 119.407502 64.0075) (end 119.300001 63.899999) (width 0.5) (layer F.Cu) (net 5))
 (segment (start 122.4075 64.0075) (end 122.365 64.0075) (width 0.5) (layer F.Cu) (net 5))
 (segment (start 122.365 64.0075) (end 119.407502 64.0075) (width 0.5) (layer F.Cu) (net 5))
 (via (at 122.365 64.0075) (size 0.5) (drill 0.3) (layers F.Cu B.Cu) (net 5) (status 30))
 (segment (start 130.048 76.832) (end 128.72 78.16) (width 0.5) (layer F.Cu) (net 12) (status 20))
 (segment (start 130.048 75.3488) (end 130.048 76.832) (width 0.5) (layer F.Cu) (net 12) (status 10))
 (via (at 120.2 67.2) (size 0.8) (drill 0.4) (layers F.Cu B.Cu) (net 6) (status 30))
 (segment (start 126.057603 73.993801) (end 122.393801 73.993801) (width 0.25) (layer F.Cu) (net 7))
 (segment (start 126.501801 74.437999) (end 126.057603 73.993801) (width 0.25) (layer F.Cu) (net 7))
 (segment (start 126.501801 76.298001) (end 126.501801 74.437999) (width 0.25) (layer F.Cu) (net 7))
 (segment (start 125.994999 78.690003) (end 125.994999 76.804803) (width 0.25) (layer F.Cu) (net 7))
 (segment (start 125.400001 79.285001) (end 125.994999 78.690003) (width 0.25) (layer F.Cu) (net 7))
 (segment (start 123.845001 79.285001) (end 125.400001 79.285001) (width 0.25) (layer F.Cu) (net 7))
 (segment (start 122.72 78.16) (end 123.845001 79.285001) (width 0.25) (layer F.Cu) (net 7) (status 10))
 (segment (start 125.994999 76.804803) (end 126.501801 76.298001) (width 0.25) (layer F.Cu) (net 7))
 (segment (start 122.393801 73.993801) (end 122.2 73.8) (width 0.25) (layer F.Cu) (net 7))
 (segment (start 122.2 73.8) (end 122.2 70.3) (width 0.25) (layer F.Cu) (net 7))
 (via (at 122.2 70.3) (size 0.8) (drill 0.4) (layers F.Cu B.Cu) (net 7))
 (segment (start 122.2 68.15) (end 122.021 67.971) (width 0.25) (layer B.Cu) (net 7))
 (segment (start 122.2 70.3) (end 122.2 68.15) (width 0.25) (layer B.Cu) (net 7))
 (segment (start 122.021 67.971) (end 121.15 67.1) (width 0.25) (layer B.Cu) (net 7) (status 20))
 (via (at 122.021 67.971) (size 0.5) (drill 0.3) (layers F.Cu B.Cu) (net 7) (status 30))
 (segment (start 126.492 69.9268) (end 123.4 73.0188) (width 0.5) (layer F.Cu) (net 1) (status 20))
 (segment (start 126.492 69.088) (end 126.492 69.9268) (width 0.5) (layer F.Cu) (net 1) (status 10))
 (segment (start 123.4 75.48) (end 120.72 78.16) (width 0.5) (layer F.Cu) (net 10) (status 30))
 (segment (start 123.4 75.4188) (end 123.4 75.48) (width 0.5) (layer F.Cu) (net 10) (status 30))
 (via (at 117.8 62.5) (size 0.8) (drill 0.4) (layers F.Cu B.Cu) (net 11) (status 30))
 (segment (start 123 66.5) (end 129.5 66.5) (width 0.5) (layer F.Cu) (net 8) (status 30))
 (segment (start 120.5 72.6) (end 121.7 72.6) (width 0.5) (layer B.Cu) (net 8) (status 10))
 (segment (start 123 71.3) (end 123 66.5) (width 0.5) (layer B.Cu) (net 8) (status 20))
 (segment (start 121.7 72.6) (end 123 71.3) (width 0.5) (layer B.Cu) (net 8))
 (segment (start 121.15 63.45) (end 121.15 64.5) (width 0.5) (layer B.Cu) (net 8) (status 20))
 (segment (start 120.3 62.6) (end 121.15 63.45) (width 0.5) (layer B.Cu) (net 8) (status 10))
 (segment (start 121.15 64.65) (end 123 66.5) (width 0.5) (layer B.Cu) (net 8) (status 30))
 (segment (start 121.15 64.5) (end 121.15 64.65) (width 0.5) (layer B.Cu) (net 8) (status 30))
 (segment (start 120.550001 65.149999) (end 126.050001 65.149999) (width 0.5) (layer F.Cu) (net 4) (status 10))
 (segment (start 120.3 65.4) (end 120.550001 65.149999) (width 0.5) (layer F.Cu) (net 4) (status 30))
 (segment (start 126.050001 65.149999) (end 127.55 63.65) (width 0.5) (layer F.Cu) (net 4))
 (segment (start 127.55 63.65) (end 127.6 63.6) (width 0.5) (layer F.Cu) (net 4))
 (via (at 127.55 63.65) (size 0.8) (drill 0.4) (layers F.Cu B.Cu) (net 4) (status 30)))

